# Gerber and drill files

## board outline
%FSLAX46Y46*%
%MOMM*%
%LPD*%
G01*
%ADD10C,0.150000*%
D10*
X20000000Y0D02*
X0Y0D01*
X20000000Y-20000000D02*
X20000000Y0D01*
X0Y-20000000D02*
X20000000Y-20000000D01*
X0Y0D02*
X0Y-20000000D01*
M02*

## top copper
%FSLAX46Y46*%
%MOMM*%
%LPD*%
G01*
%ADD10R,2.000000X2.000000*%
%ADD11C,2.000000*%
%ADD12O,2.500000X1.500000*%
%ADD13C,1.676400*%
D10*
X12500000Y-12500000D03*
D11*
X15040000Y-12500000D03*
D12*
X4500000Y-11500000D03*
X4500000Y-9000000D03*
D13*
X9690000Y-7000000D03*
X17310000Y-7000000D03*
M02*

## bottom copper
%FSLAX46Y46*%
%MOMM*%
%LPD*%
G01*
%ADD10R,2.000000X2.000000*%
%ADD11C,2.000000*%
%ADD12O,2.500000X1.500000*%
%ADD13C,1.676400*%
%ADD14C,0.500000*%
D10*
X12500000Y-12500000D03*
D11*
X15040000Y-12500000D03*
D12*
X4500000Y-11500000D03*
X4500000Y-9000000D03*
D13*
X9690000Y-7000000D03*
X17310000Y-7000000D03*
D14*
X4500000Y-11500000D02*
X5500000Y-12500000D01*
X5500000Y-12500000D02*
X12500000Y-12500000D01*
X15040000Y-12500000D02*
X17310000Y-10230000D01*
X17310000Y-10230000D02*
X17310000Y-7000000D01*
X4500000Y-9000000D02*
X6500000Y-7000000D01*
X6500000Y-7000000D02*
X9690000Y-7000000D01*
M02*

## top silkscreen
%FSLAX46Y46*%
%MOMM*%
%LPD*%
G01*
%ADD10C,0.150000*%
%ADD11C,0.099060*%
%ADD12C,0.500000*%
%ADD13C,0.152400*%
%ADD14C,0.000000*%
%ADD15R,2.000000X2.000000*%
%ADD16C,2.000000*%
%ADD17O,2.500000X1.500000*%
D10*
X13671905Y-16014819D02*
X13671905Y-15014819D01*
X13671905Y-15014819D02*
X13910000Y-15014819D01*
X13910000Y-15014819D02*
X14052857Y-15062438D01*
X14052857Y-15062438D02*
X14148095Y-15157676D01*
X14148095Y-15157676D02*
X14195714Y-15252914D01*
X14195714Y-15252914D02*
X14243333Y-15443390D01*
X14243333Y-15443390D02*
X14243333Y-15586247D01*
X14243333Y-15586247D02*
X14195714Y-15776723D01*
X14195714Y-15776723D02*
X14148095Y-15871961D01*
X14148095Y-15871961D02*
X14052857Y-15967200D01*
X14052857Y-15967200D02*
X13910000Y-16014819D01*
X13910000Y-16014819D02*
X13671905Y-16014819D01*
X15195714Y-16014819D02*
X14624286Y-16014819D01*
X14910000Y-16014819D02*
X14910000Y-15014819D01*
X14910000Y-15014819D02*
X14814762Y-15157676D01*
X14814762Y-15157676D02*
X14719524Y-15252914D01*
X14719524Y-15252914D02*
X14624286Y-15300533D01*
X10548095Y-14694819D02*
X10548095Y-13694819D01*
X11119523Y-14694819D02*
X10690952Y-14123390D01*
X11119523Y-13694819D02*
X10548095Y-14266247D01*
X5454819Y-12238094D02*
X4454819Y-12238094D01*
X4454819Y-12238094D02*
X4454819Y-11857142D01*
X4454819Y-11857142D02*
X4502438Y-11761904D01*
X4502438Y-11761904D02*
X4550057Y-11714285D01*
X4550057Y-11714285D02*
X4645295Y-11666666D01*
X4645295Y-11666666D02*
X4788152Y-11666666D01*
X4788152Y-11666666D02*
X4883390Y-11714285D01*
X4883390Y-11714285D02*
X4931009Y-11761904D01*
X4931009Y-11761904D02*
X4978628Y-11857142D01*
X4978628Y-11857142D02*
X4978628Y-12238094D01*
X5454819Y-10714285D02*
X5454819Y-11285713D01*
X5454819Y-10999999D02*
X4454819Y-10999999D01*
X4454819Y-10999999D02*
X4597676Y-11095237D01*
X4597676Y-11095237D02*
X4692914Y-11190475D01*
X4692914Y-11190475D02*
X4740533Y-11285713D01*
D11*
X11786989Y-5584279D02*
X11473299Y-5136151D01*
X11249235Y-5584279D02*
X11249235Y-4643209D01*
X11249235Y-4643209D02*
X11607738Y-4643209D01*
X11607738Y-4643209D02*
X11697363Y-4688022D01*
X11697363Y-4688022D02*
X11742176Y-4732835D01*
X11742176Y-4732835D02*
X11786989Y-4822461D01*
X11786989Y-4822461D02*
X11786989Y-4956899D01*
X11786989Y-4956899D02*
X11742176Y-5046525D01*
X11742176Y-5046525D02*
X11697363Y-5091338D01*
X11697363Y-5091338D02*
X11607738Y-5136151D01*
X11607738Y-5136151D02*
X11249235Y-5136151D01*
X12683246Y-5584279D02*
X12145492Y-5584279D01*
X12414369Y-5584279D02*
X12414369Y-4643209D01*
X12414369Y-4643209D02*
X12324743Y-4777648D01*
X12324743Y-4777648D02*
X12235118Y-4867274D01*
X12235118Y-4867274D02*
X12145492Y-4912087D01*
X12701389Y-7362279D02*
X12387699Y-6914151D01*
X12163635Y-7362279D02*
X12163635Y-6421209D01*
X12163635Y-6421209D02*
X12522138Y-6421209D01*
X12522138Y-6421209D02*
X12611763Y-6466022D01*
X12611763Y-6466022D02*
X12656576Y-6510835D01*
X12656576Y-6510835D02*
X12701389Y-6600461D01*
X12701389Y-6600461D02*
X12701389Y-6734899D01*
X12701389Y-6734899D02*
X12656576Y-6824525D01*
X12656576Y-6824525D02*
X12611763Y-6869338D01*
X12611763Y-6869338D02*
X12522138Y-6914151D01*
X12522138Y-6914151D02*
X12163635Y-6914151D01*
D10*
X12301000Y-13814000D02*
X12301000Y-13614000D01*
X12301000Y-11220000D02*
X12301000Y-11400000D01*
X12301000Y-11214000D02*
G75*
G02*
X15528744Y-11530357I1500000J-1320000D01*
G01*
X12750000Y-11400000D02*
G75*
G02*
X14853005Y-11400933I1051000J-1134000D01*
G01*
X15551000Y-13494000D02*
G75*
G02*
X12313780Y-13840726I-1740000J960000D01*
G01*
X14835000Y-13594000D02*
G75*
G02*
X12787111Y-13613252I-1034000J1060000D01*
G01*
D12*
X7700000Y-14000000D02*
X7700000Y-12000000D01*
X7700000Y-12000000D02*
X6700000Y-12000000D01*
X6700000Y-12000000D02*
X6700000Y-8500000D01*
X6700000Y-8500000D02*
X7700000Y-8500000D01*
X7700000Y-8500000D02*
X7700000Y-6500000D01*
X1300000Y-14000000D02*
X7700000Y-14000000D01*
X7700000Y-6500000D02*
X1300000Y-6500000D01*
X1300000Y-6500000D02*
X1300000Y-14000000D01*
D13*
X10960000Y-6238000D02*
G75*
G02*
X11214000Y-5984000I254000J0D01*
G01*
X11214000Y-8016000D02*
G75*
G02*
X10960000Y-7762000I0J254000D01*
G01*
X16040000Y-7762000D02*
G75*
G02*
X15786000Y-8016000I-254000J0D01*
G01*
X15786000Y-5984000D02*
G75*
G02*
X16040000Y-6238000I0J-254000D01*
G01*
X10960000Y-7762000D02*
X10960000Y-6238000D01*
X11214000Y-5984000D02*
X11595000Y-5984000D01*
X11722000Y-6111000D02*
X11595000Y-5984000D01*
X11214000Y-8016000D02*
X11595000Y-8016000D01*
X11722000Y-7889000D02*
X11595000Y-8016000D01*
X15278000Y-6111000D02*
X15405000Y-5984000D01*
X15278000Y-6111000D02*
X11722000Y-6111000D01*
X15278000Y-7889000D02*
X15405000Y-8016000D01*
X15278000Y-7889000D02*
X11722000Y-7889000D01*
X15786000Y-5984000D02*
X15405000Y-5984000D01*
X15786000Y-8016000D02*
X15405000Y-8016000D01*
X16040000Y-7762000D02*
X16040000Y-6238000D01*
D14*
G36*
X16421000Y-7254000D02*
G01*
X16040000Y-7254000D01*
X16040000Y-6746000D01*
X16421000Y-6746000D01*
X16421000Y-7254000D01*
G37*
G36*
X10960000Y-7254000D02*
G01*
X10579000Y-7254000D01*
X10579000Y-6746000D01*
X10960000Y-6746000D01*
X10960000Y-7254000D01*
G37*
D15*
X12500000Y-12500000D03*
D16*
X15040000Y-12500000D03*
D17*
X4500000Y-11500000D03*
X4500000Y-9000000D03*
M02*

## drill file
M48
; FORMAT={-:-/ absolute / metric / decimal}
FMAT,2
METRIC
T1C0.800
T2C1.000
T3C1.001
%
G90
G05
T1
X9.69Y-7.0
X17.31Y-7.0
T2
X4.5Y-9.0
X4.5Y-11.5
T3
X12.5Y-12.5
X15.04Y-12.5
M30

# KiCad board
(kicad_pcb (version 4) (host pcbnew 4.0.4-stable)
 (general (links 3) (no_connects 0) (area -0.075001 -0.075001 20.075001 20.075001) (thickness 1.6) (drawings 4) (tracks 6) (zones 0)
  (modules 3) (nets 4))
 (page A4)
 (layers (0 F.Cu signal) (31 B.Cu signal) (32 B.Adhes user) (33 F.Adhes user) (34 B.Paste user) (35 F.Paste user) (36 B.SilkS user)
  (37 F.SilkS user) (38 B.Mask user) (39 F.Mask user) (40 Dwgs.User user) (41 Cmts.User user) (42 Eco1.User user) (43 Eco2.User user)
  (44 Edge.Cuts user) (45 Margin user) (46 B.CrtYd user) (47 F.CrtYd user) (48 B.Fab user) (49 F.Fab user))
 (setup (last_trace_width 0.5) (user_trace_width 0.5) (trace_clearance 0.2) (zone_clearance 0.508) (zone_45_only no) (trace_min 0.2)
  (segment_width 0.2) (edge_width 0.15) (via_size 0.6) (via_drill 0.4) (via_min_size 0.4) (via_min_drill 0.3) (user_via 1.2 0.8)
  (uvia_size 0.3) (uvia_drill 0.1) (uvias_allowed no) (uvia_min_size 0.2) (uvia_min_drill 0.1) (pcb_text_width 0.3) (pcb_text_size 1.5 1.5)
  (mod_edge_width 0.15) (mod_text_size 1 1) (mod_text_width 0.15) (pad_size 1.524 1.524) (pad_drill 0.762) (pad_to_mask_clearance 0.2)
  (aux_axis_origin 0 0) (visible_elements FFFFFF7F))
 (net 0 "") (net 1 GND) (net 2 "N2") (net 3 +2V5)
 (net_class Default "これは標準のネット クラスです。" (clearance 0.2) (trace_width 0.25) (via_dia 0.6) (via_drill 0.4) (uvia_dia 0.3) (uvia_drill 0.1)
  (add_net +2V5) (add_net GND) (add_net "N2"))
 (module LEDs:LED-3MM (layer F.Cu) (at 12.5 12.5)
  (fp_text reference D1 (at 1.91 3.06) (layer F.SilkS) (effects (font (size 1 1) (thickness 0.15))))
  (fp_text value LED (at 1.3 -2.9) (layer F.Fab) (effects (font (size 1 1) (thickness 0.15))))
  (fp_line (start -0.199 1.314) (end -0.199 1.114) (layer F.SilkS) (width 0.15))
  (fp_line (start -0.199 -1.28) (end -0.199 -1.1) (layer F.SilkS) (width 0.15))
  (fp_arc (start 1.301 0.034) (end -0.199 -1.286) (angle 108.5) (layer F.SilkS) (width 0.15))
  (fp_arc (start 1.301 0.034) (end 0.25 -1.1) (angle 85.7) (layer F.SilkS) (width 0.15))
  (fp_arc (start 1.311 0.034) (end 3.051 0.994) (angle 110) (layer F.SilkS) (width 0.15))
  (fp_arc (start 1.301 0.034) (end 2.335 1.094) (angle 87.5) (layer F.SilkS) (width 0.15))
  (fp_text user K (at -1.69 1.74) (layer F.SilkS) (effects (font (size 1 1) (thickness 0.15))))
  (pad 1 thru_hole rect (at 0 0 90) (size 2 2) (drill 1.00076) (layers *.Cu *.Mask F.SilkS) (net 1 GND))
  (pad 2 thru_hole circle (at 2.54 0) (size 2 2) (drill 1.00076) (layers *.Cu *.Mask F.SilkS) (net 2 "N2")))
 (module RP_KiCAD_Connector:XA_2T (layer F.Cu) (at 4.5 11.5 90)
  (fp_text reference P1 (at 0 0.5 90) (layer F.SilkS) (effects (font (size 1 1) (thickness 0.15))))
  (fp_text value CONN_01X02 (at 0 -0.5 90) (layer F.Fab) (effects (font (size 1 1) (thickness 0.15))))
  (fp_line (start -2.5 3.2) (end -0.5 3.2) (layer F.SilkS) (width 0.5))
  (fp_line (start -0.5 3.2) (end -0.5 2.2) (layer F.SilkS) (width 0.5))
  (fp_line (start -0.5 2.2) (end 3 2.2) (layer F.SilkS) (width 0.5))
  (fp_line (start 3 2.2) (end 3 3.2) (layer F.SilkS) (width 0.5))
  (fp_line (start 3 3.2) (end 5 3.2) (layer F.SilkS) (width 0.5))
  (fp_line (start -2.5 -3.2) (end -2.5 3.2) (layer F.SilkS) (width 0.5))
  (fp_line (start 5 3.2) (end 5 -3.2) (layer F.SilkS) (width 0.5))
  (fp_line (start 5 -3.2) (end -2.5 -3.2) (layer F.SilkS) (width 0.5))
  (pad 2 thru_hole oval (at 0 0 90) (size 1.5 2.5) (drill 1) (layers *.Cu *.Mask F.SilkS) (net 1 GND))
  (pad 1 thru_hole oval (at 2.5 0 90) (size 1.5 2.5) (drill 1) (layers *.Cu *.Mask F.SilkS) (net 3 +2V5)))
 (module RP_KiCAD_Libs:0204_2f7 (layer F.Cu) (at 13.5 7)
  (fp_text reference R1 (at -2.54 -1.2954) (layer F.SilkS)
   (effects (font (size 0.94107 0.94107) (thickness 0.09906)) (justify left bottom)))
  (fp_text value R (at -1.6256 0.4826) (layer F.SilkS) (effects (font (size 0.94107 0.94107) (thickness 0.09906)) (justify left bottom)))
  (fp_arc (start -2.286 -0.762) (end -2.54 -0.762) (angle 90) (layer F.SilkS) (width 0.1524))
  (fp_arc (start -2.286 0.762) (end -2.54 0.762) (angle -90) (layer F.SilkS) (width 0.1524))
  (fp_arc (start 2.286 0.762) (end 2.286 1.016) (angle -90) (layer F.SilkS) (width 0.1524))
  (fp_arc (start 2.286 -0.762) (end 2.286 -1.016) (angle 90) (layer F.SilkS) (width 0.1524))
  (fp_line (start -2.54 0.762) (end -2.54 -0.762) (layer F.SilkS) (width 0.1524))
  (fp_line (start -2.286 -1.016) (end -1.905 -1.016) (layer F.SilkS) (width 0.1524))
  (fp_line (start -1.778 -0.889) (end -1.905 -1.016) (layer F.SilkS) (width 0.1524))
  (fp_line (start -2.286 1.016) (end -1.905 1.016) (layer F.SilkS) (width 0.1524))
  (fp_line (start -1.778 0.889) (end -1.905 1.016) (layer F.SilkS) (width 0.1524))
  (fp_line (start 1.778 -0.889) (end 1.905 -1.016) (layer F.SilkS) (width 0.1524))
  (fp_line (start 1.778 -0.889) (end -1.778 -0.889) (layer F.SilkS) (width 0.1524))
  (fp_line (start 1.778 0.889) (end 1.905 1.016) (layer F.SilkS) (width 0.1524))
  (fp_line (start 1.778 0.889) (end -1.778 0.889) (layer F.SilkS) (width 0.1524))
  (fp_line (start 2.286 -1.016) (end 1.905 -1.016) (layer F.SilkS) (width 0.1524))
  (fp_line (start 2.286 1.016) (end 1.905 1.016) (layer F.SilkS) (width 0.1524))
  (fp_line (start 2.54 0.762) (end 2.54 -0.762) (layer F.SilkS) (width 0.1524))
  (fp_poly (pts (xy 2.54 0.254) (xy 2.921 0.254) (xy 2.921 -0.254) (xy 2.54 -0.254)) (layer F.SilkS) (width 0))
  (fp_poly (pts (xy -2.921 0.254) (xy -2.54 0.254) (xy -2.54 -0.254) (xy -2.921 -0.254)) (layer F.SilkS) (width 0))
  (pad 1 thru_hole circle (at -3.81 0) (size 1.6764 1.6764) (drill 0.8) (layers *.Cu *.Mask) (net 3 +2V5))
  (pad 2 thru_hole circle (at 3.81 0) (size 1.6764 1.6764) (drill 0.8) (layers *.Cu *.Mask) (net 2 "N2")))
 (gr_line (start 20 0) (end 0 0) (angle 90) (layer Edge.Cuts) (width 0.15))
 (gr_line (start 20 20) (end 20 0) (angle 90) (layer Edge.Cuts) (width 0.15))
 (gr_line (start 0 20) (end 20 20) (angle 90) (layer Edge.Cuts) (width 0.15))
 (gr_line (start 0 0) (end 0 20) (angle 90) (layer Edge.Cuts) (width 0.15))
 (segment (start 4.5 11.5) (end 5.5 12.5) (width 0.5) (layer B.Cu) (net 1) (status 400000))
 (segment (start 5.5 12.5) (end 12.5 12.5) (width 0.5) (layer B.Cu) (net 1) (status 800000))
 (segment (start 15.04 12.5) (end 17.31 10.23) (width 0.5) (layer B.Cu) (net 2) (status 400000))
 (segment (start 17.31 10.23) (end 17.31 7) (width 0.5) (layer B.Cu) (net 2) (status 800000))
 (segment (start 4.5 9) (end 6.5 7) (width 0.5) (layer B.Cu) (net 3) (status 400000))
 (segment (start 6.5 7) (end 9.69 7) (width 0.5) (layer B.Cu) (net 3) (status 800000)))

